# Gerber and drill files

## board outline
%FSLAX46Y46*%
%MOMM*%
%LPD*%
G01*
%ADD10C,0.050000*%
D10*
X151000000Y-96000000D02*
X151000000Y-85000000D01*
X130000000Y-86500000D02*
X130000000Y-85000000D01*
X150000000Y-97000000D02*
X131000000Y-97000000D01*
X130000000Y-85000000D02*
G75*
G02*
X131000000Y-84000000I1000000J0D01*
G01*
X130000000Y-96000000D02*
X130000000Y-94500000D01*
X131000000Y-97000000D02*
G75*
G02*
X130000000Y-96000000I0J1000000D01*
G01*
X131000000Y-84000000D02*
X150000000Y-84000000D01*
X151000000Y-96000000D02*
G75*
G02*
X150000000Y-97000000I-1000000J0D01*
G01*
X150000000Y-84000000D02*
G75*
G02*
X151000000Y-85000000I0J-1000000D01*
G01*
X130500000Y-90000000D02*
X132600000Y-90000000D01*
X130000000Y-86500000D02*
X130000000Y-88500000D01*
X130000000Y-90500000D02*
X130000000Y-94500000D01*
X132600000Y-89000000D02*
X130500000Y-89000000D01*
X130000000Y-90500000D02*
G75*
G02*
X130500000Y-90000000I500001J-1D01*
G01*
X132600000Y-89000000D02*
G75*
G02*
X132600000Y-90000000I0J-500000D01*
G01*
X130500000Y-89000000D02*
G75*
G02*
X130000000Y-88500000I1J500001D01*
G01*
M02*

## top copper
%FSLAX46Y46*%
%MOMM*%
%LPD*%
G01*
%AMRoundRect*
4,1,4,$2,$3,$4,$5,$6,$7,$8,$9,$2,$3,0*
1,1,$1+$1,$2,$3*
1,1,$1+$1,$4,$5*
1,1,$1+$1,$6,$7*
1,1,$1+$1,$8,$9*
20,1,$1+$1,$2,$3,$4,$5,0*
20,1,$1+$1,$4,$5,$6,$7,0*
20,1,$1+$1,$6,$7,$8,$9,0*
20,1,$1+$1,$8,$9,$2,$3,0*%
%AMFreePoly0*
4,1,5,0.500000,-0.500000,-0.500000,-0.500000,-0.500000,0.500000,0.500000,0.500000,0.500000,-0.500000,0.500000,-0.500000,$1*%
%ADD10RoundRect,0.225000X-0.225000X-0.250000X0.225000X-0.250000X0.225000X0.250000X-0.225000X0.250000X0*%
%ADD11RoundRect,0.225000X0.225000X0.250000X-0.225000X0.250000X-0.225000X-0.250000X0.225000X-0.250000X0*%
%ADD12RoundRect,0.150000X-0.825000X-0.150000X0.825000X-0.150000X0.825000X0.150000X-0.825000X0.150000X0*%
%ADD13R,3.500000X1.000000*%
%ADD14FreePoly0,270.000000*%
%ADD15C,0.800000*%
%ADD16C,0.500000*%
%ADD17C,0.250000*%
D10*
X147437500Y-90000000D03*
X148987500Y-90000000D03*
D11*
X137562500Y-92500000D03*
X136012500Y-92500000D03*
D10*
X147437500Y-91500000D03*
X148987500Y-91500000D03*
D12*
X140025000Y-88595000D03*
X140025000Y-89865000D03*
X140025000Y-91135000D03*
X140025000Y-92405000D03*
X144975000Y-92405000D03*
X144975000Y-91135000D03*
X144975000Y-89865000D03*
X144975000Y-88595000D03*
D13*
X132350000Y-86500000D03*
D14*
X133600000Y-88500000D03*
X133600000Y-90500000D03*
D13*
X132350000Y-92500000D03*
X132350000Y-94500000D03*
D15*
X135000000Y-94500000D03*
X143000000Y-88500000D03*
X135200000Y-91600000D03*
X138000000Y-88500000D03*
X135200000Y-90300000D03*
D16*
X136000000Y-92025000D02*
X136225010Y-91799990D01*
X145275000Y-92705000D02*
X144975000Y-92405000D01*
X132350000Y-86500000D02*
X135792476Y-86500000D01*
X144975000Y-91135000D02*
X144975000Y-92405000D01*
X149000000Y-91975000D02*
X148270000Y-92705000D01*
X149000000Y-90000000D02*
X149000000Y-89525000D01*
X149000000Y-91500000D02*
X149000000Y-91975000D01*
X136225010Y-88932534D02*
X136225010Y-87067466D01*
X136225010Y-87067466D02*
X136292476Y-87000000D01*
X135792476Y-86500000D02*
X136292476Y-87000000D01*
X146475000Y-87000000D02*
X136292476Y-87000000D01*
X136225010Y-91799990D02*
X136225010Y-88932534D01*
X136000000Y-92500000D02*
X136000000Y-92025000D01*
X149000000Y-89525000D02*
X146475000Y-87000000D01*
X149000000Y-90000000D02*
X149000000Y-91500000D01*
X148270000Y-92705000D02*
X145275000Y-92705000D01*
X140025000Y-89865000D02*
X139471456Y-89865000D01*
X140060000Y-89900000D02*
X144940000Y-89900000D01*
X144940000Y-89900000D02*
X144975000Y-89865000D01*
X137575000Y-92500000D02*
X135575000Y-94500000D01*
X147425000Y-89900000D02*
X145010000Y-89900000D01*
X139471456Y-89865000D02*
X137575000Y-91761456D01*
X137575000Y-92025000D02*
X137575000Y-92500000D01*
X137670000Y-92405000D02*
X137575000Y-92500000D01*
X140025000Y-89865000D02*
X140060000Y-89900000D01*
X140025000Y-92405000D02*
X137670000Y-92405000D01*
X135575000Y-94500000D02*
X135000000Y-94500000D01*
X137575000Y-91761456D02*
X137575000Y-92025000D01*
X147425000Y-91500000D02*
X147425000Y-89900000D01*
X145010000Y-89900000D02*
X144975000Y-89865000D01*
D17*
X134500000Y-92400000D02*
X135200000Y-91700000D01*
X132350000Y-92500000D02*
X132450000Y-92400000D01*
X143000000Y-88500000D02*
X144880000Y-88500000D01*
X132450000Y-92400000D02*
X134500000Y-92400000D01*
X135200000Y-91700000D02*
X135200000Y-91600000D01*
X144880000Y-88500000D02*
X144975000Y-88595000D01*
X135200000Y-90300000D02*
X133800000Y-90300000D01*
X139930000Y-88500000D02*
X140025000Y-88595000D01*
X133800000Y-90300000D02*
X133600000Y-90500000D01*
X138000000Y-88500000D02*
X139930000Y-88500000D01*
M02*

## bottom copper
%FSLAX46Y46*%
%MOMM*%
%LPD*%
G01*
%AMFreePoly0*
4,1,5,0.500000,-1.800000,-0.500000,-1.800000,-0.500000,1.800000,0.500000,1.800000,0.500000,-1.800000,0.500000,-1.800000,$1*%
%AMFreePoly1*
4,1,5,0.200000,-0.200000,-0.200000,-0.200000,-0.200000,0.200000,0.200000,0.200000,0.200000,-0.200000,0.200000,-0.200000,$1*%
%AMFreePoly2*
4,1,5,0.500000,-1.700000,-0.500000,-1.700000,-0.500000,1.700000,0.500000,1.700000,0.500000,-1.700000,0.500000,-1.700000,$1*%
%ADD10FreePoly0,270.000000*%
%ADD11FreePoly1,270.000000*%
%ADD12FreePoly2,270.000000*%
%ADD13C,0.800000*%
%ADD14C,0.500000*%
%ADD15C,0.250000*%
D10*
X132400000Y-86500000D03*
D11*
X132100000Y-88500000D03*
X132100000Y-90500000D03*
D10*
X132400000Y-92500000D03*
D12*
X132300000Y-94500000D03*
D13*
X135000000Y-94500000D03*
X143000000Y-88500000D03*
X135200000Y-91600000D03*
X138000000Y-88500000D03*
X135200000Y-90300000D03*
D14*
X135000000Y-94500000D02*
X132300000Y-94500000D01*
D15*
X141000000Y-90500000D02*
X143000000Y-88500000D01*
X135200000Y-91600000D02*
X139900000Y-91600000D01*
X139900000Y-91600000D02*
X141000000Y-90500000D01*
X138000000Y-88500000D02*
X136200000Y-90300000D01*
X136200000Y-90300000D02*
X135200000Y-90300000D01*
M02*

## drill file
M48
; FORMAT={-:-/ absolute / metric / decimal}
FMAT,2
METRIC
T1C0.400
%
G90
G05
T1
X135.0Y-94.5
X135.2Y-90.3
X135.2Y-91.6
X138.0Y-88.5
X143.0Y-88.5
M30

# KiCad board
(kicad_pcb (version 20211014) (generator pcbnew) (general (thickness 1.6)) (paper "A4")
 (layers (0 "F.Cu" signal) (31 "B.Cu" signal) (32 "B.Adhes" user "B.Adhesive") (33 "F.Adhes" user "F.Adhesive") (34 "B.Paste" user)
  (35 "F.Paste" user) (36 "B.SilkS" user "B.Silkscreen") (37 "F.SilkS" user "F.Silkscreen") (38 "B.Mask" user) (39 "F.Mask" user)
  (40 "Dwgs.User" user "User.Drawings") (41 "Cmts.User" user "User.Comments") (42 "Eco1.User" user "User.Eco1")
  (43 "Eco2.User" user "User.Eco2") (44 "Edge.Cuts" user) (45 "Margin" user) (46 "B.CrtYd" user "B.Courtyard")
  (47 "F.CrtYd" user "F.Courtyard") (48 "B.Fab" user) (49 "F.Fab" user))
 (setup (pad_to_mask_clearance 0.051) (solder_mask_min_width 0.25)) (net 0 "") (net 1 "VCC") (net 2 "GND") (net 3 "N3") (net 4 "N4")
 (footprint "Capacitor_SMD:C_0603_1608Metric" (layer "F.Cu") (at 148.2125 90)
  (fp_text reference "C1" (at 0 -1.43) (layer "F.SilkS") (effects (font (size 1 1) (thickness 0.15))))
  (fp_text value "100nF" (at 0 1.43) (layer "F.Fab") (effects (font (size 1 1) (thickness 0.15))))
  (pad "1" smd roundrect locked (at -0.775 0) (size 0.9 0.95) (layers "F.Cu" "F.Paste" "F.Mask") (roundrect_rratio 0.25) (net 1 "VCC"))
  (pad "2" smd roundrect locked (at 0.775 0) (size 0.9 0.95) (layers "F.Cu" "F.Paste" "F.Mask") (roundrect_rratio 0.25) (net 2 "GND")))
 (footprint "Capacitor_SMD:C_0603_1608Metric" (layer "F.Cu") (at 136.7875 92.5 180)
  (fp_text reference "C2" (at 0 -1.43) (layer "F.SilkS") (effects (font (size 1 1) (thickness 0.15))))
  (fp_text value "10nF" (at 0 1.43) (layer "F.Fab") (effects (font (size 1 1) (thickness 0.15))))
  (pad "1" smd roundrect locked (at -0.775 0 180) (size 0.9 0.95) (layers "F.Cu" "F.Paste" "F.Mask") (roundrect_rratio 0.25) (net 1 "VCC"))
  (pad "2" smd roundrect locked (at 0.775 0 180) (size 0.9 0.95) (layers "F.Cu" "F.Paste" "F.Mask") (roundrect_rratio 0.25) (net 2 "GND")))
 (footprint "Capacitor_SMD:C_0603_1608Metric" (layer "F.Cu") (at 148.2125 91.5)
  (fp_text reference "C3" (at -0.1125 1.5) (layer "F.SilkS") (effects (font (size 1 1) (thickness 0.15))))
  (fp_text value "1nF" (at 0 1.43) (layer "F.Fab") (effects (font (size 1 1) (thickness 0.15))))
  (pad "1" smd roundrect locked (at -0.775 0) (size 0.9 0.95) (layers "F.Cu" "F.Paste" "F.Mask") (roundrect_rratio 0.25) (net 1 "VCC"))
  (pad "2" smd roundrect locked (at 0.775 0) (size 0.9 0.95) (layers "F.Cu" "F.Paste" "F.Mask") (roundrect_rratio 0.25) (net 2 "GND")))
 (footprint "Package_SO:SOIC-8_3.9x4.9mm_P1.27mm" (layer "F.Cu") (at 142.5 90.5)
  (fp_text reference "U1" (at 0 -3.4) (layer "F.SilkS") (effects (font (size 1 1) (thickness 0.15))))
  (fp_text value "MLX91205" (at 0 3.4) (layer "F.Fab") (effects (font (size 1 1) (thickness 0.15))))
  (pad "1" smd roundrect locked (at -2.475 -1.905) (size 1.95 0.6) (layers "F.Cu" "F.Paste" "F.Mask") (roundrect_rratio 0.25) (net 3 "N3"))
  (pad "2" smd roundrect locked (at -2.475 -0.635) (size 1.95 0.6) (layers "F.Cu" "F.Paste" "F.Mask") (roundrect_rratio 0.25) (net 1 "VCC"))
  (pad "3" smd roundrect locked (at -2.475 0.635) (size 1.95 0.6) (layers "F.Cu" "F.Paste" "F.Mask") (roundrect_rratio 0.25))
  (pad "4" smd roundrect locked (at -2.475 1.905) (size 1.95 0.6) (layers "F.Cu" "F.Paste" "F.Mask") (roundrect_rratio 0.25) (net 1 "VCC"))
  (pad "5" smd roundrect locked (at 2.475 1.905) (size 1.95 0.6) (layers "F.Cu" "F.Paste" "F.Mask") (roundrect_rratio 0.25) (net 2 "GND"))
  (pad "6" smd roundrect locked (at 2.475 0.635) (size 1.95 0.6) (layers "F.Cu" "F.Paste" "F.Mask") (roundrect_rratio 0.25) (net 2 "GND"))
  (pad "7" smd roundrect locked (at 2.475 -0.635) (size 1.95 0.6) (layers "F.Cu" "F.Paste" "F.Mask") (roundrect_rratio 0.25) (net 1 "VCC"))
  (pad "8" smd roundrect locked (at 2.475 -1.905) (size 1.95 0.6) (layers "F.Cu" "F.Paste" "F.Mask") (roundrect_rratio 0.25) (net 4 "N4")))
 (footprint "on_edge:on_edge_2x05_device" (layer "F.Cu") (at 130 90.5 -90)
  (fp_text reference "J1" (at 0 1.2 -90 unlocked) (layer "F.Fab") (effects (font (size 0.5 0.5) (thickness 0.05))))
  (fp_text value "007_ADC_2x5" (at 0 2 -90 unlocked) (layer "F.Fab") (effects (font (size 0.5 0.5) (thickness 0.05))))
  (fp_line (start -0.5 -0.5) (end -0.5 -2.6) (layer "Edge.Cuts") (width 0.05))
  (fp_line (start -4 0) (end -2 0) (layer "Edge.Cuts") (width 0.05))
  (fp_line (start 0 0) (end 4 0) (layer "Edge.Cuts") (width 0.05))
  (fp_line (start -1.5 -2.6) (end -1.5 -0.5) (layer "Edge.Cuts") (width 0.05))
  (fp_arc (start 0 0) (mid -0.353553 -0.146447) (end -0.5 -0.5) (layer "Edge.Cuts") (width 0.05))
  (fp_arc (start -1.5 -2.6) (mid -1 -3.1) (end -0.5 -2.6) (layer "Edge.Cuts") (width 0.05))
  (fp_arc (start -1.5 -0.5) (mid -1.646447 -0.146447) (end -2 0) (layer "Edge.Cuts") (width 0.05))
  (pad "1" smd rect locked (at -4 -2.35 90) (size 1 3.5) (layers "F.Cu" "F.Mask") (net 2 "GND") (zone_connect 0))
  (pad "2" smd custom locked (at -2 -3.6 270) (size 1 1) (layers "F.Cu" "F.Mask") (zone_connect 0)
   (options (clearance outline) (anchor rect)) (primitives))
  (pad "3" smd custom locked (at 0 -3.6 270) (size 1 1) (layers "F.Cu" "F.Mask") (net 3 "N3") (zone_connect 0)
   (options (clearance outline) (anchor rect)) (primitives))
  (pad "4" smd rect locked (at 2 -2.35 90) (size 1 3.5) (layers "F.Cu" "F.Mask") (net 4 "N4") (zone_connect 0))
  (pad "5" smd rect locked (at 4 -2.35 90) (size 1 3.5) (layers "F.Cu" "F.Mask") (zone_connect 0))
  (pad "6" smd custom locked (at -4 -2.4 270) (size 1 3.6) (layers "B.Cu" "B.Mask") (zone_connect 0)
   (options (clearance outline) (anchor rect)) (primitives))
  (pad "7" smd custom locked (at -2 -2.1 270) (size 0.4 0.4) (layers "B.Cu" "B.Mask") (zone_connect 0)
   (options (clearance outline) (anchor rect)) (primitives))
  (pad "8" smd custom locked (at 0 -2.1 270) (size 0.4 0.4) (layers "B.Cu" "B.Mask") (zone_connect 0)
   (options (clearance outline) (anchor rect)) (primitives))
  (pad "9" smd custom locked (at 2 -2.4 270) (size 1 3.6) (layers "B.Cu" "B.Mask") (zone_connect 0)
   (options (clearance outline) (anchor rect)) (primitives))
  (pad "10" smd custom locked (at 4 -2.3 270) (size 1 3.4) (layers "B.Cu" "B.Mask") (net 1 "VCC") (zone_connect 0)
   (options (clearance outline) (anchor rect)) (primitives)))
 (gr_line (start 151 96) (end 151 85) (layer "Edge.Cuts") (width 0.05))
 (gr_line (start 130 86.5) (end 130 85) (layer "Edge.Cuts") (width 0.05))
 (gr_line (start 150 97) (end 131 97) (layer "Edge.Cuts") (width 0.05))
 (gr_arc (start 130 85) (mid 130.292893 84.292893) (end 131 84) (layer "Edge.Cuts") (width 0.05))
 (gr_line (start 130 96) (end 130 94.5) (layer "Edge.Cuts") (width 0.05))
 (gr_arc (start 131 97) (mid 130.292893 96.707107) (end 130 96) (layer "Edge.Cuts") (width 0.05))
 (gr_line (start 131 84) (end 150 84) (layer "Edge.Cuts") (width 0.05))
 (gr_arc (start 151 96) (mid 150.707107 96.707107) (end 150 97) (layer "Edge.Cuts") (width 0.05))
 (gr_arc (start 150 84) (mid 150.707107 84.292893) (end 151 85) (layer "Edge.Cuts") (width 0.05))
 (segment (start 136 92.025) (end 136.22501 91.79999) (width 0.5) (layer "F.Cu") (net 2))
 (segment (start 145.275 92.705) (end 144.975 92.405) (width 0.5) (layer "F.Cu") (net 2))
 (segment (start 132.35 86.5) (end 135.792476 86.5) (width 0.5) (layer "F.Cu") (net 2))
 (segment (start 144.975 91.135) (end 144.975 92.405) (width 0.5) (layer "F.Cu") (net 2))
 (segment (start 149 91.975) (end 148.27 92.705) (width 0.5) (layer "F.Cu") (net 2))
 (segment (start 149 90) (end 149 89.525) (width 0.5) (layer "F.Cu") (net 2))
 (segment (start 149 91.5) (end 149 91.975) (width 0.5) (layer "F.Cu") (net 2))
 (segment (start 136.22501 88.932534) (end 136.22501 87.067466) (width 0.5) (layer "F.Cu") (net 2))
 (segment (start 136.22501 87.067466) (end 136.292476 87) (width 0.5) (layer "F.Cu") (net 2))
 (segment (start 135.792476 86.5) (end 136.292476 87) (width 0.5) (layer "F.Cu") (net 2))
 (segment (start 146.475 87) (end 136.292476 87) (width 0.5) (layer "F.Cu") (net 2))
 (segment (start 136.22501 91.79999) (end 136.22501 88.932534) (width 0.5) (layer "F.Cu") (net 2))
 (segment (start 136 92.5) (end 136 92.025) (width 0.5) (layer "F.Cu") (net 2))
 (segment (start 149 89.525) (end 146.475 87) (width 0.5) (layer "F.Cu") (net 2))
 (segment (start 149 90) (end 149 91.5) (width 0.5) (layer "F.Cu") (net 2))
 (segment (start 148.27 92.705) (end 145.275 92.705) (width 0.5) (layer "F.Cu") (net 2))
 (segment (start 140.025 89.865) (end 139.471456 89.865) (width 0.5) (layer "F.Cu") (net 1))
 (segment (start 140.06 89.9) (end 144.94 89.9) (width 0.5) (layer "F.Cu") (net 1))
 (segment (start 144.94 89.9) (end 144.975 89.865) (width 0.5) (layer "F.Cu") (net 1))
 (segment (start 137.575 92.5) (end 135.575 94.5) (width 0.5) (layer "F.Cu") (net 1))
 (segment (start 147.425 89.9) (end 145.01 89.9) (width 0.5) (layer "F.Cu") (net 1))
 (segment (start 139.471456 89.865) (end 137.575 91.761456) (width 0.5) (layer "F.Cu") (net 1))
 (segment (start 137.575 92.025) (end 137.575 92.5) (width 0.5) (layer "F.Cu") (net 1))
 (segment (start 137.67 92.405) (end 137.575 92.5) (width 0.5) (layer "F.Cu") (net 1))
 (segment (start 140.025 89.865) (end 140.06 89.9) (width 0.5) (layer "F.Cu") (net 1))
 (segment (start 140.025 92.405) (end 137.67 92.405) (width 0.5) (layer "F.Cu") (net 1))
 (segment (start 135.575 94.5) (end 135 94.5) (width 0.5) (layer "F.Cu") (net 1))
 (segment (start 137.575 91.761456) (end 137.575 92.025) (width 0.5) (layer "F.Cu") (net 1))
 (segment (start 147.425 91.5) (end 147.425 89.9) (width 0.5) (layer "F.Cu") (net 1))
 (segment (start 145.01 89.9) (end 144.975 89.865) (width 0.5) (layer "F.Cu") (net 1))
 (via (at 135 94.5) (size 0.8) (drill 0.4) (layers "F.Cu" "B.Cu") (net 1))
 (segment (start 135 94.5) (end 132.3 94.5) (width 0.5) (layer "B.Cu") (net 1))
 (segment (start 134.5 92.4) (end 135.2 91.7) (width 0.25) (layer "F.Cu") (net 4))
 (segment (start 132.35 92.5) (end 132.45 92.4) (width 0.25) (layer "F.Cu") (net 4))
 (segment (start 143 88.5) (end 144.88 88.5) (width 0.25) (layer "F.Cu") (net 4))
 (segment (start 132.45 92.4) (end 134.5 92.4) (width 0.25) (layer "F.Cu") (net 4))
 (segment (start 135.2 91.7) (end 135.2 91.6) (width 0.25) (layer "F.Cu") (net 4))
 (segment (start 144.88 88.5) (end 144.975 88.595) (width 0.25) (layer "F.Cu") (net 4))
 (via (at 143 88.5) (size 0.8) (drill 0.4) (layers "F.Cu" "B.Cu") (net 4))
 (via (at 135.2 91.6) (size 0.8) (drill 0.4) (layers "F.Cu" "B.Cu") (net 4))
 (segment (start 141 90.5) (end 143 88.5) (width 0.25) (layer "B.Cu") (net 4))
 (segment (start 135.2 91.6) (end 139.9 91.6) (width 0.25) (layer "B.Cu") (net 4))
 (segment (start 139.9 91.6) (end 141 90.5) (width 0.25) (layer "B.Cu") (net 4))
 (segment (start 135.2 90.3) (end 133.8 90.3) (width 0.25) (layer "F.Cu") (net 3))
 (segment (start 139.93 88.5) (end 140.025 88.595) (width 0.25) (layer "F.Cu") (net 3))
 (segment (start 133.8 90.3) (end 133.6 90.5) (width 0.25) (layer "F.Cu") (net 3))
 (segment (start 138 88.5) (end 139.93 88.5) (width 0.25) (layer "F.Cu") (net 3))
 (via (at 138 88.5) (size 0.8) (drill 0.4) (layers "F.Cu" "B.Cu") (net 3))
 (via (at 135.2 90.3) (size 0.8) (drill 0.4) (layers "F.Cu" "B.Cu") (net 3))
 (segment (start 138 88.5) (end 136.2 90.3) (width 0.25) (layer "B.Cu") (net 3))
 (segment (start 136.2 90.3) (end 135.2 90.3) (width 0.25) (layer "B.Cu") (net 3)))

